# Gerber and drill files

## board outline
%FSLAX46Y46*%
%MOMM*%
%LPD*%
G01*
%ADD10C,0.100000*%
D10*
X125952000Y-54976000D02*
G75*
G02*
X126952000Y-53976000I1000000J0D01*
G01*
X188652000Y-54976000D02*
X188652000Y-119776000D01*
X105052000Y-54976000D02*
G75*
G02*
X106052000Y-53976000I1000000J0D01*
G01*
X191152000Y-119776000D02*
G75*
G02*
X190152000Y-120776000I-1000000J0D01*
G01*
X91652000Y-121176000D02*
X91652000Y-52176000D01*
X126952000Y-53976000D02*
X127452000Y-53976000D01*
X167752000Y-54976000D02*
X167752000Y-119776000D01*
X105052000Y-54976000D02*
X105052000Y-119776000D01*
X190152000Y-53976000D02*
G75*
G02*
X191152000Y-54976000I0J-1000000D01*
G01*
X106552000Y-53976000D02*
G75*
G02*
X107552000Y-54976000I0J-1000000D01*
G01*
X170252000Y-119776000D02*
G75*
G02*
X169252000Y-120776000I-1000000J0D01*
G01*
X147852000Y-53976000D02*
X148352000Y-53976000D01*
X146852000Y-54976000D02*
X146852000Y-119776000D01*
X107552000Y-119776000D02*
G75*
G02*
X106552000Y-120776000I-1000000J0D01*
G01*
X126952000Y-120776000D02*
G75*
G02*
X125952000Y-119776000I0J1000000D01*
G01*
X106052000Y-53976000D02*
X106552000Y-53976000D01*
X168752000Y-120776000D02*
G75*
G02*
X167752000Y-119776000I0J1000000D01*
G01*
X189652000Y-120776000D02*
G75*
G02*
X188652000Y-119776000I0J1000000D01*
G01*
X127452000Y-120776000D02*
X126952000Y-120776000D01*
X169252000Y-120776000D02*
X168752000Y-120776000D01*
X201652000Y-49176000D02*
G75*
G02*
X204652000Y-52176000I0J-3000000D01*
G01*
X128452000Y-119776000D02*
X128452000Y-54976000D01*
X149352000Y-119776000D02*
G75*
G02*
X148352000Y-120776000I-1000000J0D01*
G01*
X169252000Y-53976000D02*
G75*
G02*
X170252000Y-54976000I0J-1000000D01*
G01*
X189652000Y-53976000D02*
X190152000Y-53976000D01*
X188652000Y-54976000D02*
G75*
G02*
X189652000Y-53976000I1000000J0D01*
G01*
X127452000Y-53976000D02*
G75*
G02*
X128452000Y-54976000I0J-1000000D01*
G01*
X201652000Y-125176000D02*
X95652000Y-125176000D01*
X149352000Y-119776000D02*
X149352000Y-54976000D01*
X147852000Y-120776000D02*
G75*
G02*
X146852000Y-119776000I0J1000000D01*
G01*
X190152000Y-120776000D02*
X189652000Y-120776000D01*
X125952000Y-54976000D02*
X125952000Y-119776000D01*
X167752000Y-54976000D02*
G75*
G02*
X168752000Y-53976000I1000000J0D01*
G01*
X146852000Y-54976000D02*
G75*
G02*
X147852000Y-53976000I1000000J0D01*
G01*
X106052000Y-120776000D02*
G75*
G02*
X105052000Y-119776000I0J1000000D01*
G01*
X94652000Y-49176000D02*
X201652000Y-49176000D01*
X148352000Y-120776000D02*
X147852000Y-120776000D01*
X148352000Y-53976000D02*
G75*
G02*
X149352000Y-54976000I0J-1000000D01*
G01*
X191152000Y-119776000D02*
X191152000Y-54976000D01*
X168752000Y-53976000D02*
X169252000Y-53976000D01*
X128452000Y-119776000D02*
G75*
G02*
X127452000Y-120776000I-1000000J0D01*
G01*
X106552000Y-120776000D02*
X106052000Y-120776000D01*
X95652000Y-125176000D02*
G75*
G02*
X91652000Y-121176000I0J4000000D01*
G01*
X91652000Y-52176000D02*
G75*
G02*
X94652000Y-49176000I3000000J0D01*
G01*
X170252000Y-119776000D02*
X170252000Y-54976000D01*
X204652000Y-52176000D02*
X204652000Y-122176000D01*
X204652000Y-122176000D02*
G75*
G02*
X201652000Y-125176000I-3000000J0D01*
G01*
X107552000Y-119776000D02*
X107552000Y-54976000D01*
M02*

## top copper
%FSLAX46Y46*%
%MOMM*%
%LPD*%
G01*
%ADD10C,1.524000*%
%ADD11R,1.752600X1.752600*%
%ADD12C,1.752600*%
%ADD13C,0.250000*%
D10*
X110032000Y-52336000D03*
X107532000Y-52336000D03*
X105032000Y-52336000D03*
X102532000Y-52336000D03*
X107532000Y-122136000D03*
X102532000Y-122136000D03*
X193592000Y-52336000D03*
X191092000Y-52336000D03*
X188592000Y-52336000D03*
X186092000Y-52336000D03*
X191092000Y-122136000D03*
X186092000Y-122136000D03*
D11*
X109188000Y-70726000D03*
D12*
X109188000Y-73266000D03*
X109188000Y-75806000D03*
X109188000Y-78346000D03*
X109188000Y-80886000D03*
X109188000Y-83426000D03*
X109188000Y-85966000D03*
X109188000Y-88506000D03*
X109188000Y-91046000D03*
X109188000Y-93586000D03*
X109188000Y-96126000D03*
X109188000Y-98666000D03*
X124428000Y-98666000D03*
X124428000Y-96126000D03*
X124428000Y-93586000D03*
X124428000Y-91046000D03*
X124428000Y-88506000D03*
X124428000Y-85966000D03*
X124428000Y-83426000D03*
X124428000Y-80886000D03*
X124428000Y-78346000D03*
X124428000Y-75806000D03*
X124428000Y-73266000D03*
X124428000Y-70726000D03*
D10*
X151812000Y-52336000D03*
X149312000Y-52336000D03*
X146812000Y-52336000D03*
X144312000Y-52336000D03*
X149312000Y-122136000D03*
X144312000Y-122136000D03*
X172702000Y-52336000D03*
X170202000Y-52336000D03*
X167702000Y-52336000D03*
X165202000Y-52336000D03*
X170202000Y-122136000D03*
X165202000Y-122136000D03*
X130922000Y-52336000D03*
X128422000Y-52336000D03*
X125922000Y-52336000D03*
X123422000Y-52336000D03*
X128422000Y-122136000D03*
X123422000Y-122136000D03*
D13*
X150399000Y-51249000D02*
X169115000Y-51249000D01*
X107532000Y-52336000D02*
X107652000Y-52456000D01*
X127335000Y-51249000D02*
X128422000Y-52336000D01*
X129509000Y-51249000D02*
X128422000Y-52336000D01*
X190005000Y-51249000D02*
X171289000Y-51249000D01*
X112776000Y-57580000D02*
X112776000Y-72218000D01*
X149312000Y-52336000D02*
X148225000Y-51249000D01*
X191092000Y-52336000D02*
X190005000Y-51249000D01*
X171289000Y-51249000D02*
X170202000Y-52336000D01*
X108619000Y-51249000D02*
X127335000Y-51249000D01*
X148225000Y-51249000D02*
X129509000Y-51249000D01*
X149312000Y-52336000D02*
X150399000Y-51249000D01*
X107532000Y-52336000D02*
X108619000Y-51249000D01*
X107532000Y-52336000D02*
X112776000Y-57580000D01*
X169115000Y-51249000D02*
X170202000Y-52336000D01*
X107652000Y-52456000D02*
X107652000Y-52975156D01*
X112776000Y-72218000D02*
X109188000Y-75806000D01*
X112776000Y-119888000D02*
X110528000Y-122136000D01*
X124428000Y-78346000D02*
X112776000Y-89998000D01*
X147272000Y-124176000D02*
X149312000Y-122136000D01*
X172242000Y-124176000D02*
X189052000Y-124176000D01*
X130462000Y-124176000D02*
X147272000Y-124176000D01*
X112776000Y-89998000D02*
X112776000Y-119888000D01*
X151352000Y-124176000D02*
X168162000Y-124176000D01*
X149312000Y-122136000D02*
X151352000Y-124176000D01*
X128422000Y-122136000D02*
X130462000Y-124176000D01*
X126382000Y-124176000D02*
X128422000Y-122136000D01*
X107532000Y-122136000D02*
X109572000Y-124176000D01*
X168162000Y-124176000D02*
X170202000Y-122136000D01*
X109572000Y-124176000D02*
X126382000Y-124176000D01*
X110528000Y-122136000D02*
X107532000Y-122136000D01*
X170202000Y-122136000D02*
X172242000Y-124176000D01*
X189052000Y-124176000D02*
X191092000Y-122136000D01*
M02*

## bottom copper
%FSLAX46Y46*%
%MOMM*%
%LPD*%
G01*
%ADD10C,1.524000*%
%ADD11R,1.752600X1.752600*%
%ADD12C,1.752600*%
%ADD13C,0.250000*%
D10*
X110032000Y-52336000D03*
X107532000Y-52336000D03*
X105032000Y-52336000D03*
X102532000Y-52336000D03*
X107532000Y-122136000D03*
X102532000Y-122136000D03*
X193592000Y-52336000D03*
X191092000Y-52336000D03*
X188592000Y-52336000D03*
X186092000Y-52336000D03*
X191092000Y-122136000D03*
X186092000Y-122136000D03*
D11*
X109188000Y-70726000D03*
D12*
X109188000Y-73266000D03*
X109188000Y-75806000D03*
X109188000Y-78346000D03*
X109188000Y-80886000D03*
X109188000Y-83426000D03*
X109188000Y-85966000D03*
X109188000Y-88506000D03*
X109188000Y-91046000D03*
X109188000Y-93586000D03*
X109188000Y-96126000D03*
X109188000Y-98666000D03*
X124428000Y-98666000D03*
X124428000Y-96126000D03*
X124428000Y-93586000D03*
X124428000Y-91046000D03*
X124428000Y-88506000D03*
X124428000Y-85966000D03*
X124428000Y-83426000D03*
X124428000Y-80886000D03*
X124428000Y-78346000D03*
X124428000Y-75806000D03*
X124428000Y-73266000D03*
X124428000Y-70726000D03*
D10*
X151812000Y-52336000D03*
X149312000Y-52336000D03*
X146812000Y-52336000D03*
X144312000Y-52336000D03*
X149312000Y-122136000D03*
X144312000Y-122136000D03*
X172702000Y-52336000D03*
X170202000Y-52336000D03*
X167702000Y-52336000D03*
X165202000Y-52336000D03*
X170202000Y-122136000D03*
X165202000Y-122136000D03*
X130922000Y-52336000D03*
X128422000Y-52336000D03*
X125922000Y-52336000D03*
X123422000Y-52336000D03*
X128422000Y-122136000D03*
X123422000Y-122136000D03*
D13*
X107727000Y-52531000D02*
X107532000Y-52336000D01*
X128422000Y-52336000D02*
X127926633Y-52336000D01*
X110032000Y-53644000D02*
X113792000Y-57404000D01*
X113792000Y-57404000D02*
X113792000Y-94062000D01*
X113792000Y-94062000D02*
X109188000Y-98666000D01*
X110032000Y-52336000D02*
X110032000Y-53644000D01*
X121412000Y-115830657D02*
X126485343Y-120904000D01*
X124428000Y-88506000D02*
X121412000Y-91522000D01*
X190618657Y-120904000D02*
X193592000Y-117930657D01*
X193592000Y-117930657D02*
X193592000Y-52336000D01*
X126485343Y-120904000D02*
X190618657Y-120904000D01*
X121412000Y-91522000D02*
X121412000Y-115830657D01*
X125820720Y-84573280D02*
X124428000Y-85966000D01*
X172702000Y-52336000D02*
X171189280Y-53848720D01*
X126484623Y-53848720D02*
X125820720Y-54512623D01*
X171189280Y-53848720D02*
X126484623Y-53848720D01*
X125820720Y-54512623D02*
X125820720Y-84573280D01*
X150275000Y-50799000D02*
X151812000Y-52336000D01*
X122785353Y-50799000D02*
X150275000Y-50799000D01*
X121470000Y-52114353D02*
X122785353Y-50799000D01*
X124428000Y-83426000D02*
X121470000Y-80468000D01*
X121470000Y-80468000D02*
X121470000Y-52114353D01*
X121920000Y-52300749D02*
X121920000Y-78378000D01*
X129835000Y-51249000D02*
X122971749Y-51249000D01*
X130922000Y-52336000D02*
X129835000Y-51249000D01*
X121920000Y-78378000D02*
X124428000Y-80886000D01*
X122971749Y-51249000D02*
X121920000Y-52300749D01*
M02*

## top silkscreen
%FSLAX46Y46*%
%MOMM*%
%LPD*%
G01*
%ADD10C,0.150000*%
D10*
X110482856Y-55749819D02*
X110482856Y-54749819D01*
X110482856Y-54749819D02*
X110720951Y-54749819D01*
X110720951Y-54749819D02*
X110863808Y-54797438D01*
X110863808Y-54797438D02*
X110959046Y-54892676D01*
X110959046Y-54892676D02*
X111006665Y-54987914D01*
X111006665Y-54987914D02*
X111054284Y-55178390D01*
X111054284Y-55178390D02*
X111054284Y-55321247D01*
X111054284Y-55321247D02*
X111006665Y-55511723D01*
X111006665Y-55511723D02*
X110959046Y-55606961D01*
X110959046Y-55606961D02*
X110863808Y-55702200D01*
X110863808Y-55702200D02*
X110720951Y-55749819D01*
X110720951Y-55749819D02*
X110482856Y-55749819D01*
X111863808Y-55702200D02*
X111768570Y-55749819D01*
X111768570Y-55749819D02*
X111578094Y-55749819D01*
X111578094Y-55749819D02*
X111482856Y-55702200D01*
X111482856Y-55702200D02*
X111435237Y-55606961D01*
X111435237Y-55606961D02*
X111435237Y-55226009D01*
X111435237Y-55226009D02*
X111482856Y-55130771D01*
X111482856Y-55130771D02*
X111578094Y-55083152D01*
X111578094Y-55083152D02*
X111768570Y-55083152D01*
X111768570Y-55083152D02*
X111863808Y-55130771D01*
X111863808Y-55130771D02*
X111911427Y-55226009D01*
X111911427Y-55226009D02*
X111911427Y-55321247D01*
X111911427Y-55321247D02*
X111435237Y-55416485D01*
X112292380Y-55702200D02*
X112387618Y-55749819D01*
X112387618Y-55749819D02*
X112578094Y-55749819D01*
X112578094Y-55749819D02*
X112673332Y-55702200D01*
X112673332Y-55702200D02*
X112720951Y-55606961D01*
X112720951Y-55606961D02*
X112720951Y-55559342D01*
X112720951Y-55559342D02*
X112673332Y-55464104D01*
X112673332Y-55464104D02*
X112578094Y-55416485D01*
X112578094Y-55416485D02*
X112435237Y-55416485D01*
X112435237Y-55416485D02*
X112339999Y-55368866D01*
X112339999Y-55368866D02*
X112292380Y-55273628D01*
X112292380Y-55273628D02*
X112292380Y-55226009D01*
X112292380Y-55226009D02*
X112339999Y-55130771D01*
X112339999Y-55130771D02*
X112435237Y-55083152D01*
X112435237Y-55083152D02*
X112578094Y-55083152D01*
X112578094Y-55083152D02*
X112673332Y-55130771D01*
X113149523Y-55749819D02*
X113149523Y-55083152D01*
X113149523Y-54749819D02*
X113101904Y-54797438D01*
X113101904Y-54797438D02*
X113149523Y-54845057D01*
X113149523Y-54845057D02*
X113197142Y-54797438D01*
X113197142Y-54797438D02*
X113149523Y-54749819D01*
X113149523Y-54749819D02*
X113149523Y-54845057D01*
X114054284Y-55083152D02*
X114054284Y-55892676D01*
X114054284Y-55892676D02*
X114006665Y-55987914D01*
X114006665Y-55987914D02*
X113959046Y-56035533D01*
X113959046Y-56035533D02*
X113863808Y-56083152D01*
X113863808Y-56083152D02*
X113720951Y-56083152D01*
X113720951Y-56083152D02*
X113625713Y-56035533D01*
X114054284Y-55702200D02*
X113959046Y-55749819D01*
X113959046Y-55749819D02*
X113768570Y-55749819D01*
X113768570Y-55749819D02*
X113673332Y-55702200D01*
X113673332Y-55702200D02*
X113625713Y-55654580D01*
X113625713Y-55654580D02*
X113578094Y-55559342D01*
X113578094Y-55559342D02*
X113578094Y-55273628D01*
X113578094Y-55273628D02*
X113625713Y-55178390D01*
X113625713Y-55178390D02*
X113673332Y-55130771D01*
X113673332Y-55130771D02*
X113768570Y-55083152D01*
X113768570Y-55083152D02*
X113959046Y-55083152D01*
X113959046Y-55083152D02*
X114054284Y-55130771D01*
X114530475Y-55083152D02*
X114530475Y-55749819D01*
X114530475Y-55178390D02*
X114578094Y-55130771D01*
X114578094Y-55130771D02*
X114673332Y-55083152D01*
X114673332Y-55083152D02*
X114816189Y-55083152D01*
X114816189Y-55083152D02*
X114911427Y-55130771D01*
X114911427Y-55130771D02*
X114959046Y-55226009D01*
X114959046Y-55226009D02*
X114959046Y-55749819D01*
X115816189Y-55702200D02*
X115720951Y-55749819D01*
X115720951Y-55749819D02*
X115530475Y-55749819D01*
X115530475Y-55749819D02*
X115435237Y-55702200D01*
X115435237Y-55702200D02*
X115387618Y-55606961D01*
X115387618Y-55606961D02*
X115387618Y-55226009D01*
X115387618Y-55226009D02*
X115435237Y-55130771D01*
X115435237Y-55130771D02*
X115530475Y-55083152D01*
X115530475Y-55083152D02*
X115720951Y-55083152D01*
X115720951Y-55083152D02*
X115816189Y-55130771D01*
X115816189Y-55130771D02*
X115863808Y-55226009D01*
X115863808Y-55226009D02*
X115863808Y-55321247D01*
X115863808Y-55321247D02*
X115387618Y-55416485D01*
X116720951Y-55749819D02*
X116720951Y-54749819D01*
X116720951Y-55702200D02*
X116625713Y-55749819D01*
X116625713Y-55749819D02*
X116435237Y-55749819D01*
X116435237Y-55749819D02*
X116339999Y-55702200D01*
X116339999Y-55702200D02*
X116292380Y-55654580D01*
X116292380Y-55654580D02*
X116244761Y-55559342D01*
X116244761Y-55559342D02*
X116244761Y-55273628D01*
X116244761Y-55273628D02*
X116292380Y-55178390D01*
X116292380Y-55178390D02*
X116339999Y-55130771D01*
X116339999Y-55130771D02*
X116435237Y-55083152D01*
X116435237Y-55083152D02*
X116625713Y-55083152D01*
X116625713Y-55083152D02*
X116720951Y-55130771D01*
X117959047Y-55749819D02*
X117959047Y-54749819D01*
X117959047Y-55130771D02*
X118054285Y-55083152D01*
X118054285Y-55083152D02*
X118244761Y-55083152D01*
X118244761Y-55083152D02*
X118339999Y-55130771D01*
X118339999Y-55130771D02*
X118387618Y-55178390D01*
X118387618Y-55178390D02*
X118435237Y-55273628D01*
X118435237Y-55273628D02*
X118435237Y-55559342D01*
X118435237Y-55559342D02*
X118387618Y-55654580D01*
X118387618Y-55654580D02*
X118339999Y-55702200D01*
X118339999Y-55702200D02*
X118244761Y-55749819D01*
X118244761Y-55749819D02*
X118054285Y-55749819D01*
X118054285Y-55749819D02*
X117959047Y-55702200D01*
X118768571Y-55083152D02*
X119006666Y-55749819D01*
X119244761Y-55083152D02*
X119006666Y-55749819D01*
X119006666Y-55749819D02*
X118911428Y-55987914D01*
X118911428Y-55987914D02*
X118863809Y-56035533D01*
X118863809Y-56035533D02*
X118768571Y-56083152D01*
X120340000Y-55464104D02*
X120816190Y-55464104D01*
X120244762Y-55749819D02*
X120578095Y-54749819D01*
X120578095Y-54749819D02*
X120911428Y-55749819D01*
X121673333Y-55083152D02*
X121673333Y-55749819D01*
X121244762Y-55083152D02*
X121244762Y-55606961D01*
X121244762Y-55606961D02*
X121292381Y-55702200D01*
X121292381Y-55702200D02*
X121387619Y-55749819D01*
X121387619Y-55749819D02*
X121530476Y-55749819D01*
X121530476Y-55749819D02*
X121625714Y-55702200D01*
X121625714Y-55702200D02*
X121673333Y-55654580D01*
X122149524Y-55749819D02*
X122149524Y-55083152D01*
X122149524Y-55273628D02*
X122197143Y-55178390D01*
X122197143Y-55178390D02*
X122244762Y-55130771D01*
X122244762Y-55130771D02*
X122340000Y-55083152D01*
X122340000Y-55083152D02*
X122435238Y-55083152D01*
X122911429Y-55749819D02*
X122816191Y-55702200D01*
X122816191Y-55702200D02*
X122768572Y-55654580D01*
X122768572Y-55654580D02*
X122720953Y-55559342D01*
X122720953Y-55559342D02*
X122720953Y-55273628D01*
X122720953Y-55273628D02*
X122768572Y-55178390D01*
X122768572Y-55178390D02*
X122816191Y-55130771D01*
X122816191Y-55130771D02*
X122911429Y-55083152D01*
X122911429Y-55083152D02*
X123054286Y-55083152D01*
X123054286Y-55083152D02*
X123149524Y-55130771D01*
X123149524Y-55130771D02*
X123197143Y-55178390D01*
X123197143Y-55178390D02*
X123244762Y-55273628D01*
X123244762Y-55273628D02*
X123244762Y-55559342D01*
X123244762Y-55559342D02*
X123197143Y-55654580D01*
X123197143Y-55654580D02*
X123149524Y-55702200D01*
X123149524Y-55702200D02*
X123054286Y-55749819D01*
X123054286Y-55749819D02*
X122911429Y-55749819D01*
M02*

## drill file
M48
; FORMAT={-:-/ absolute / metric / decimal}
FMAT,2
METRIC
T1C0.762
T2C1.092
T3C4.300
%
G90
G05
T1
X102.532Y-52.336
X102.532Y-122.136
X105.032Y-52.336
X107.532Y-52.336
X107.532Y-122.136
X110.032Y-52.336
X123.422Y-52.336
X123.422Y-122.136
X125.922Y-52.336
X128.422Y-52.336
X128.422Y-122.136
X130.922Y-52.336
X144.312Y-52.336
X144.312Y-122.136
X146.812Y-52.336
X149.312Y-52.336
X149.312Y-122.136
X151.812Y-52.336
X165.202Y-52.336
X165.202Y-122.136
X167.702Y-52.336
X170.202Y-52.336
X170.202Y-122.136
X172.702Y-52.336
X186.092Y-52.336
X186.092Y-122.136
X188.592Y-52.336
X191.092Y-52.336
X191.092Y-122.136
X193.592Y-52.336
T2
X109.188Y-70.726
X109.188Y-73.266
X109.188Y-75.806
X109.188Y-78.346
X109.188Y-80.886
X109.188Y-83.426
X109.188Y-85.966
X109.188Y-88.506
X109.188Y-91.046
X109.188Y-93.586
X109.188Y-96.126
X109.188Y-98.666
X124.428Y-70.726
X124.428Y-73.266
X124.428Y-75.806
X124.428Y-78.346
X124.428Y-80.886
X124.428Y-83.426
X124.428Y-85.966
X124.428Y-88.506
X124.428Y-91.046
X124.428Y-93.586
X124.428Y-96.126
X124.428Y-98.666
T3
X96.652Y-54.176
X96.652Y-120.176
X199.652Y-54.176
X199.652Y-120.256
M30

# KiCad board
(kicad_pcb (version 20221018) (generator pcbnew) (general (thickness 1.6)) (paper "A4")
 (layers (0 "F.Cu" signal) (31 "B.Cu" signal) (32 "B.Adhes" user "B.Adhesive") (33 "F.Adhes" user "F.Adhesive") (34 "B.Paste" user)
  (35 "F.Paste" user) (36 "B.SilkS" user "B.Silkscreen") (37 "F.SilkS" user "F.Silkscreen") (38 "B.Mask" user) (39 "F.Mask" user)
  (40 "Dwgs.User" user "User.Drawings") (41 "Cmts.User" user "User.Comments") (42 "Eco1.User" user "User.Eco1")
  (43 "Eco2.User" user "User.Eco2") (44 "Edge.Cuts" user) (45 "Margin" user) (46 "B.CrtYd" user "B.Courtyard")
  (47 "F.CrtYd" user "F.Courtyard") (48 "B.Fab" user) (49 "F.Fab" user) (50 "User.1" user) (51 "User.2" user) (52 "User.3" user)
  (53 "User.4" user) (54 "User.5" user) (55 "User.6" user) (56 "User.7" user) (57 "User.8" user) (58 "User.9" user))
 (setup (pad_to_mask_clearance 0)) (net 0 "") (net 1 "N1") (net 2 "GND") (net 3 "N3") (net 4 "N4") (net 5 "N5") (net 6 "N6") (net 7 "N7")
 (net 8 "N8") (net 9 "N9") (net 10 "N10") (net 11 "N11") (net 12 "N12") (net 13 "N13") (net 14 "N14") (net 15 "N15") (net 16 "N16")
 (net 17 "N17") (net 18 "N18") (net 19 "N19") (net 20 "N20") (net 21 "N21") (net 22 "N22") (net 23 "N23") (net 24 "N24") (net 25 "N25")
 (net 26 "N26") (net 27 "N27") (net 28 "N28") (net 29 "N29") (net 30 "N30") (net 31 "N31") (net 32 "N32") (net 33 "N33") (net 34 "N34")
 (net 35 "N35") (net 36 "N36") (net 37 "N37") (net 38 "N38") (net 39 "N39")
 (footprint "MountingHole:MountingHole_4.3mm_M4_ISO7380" (layer "F.Cu") (at 199.652 120.256)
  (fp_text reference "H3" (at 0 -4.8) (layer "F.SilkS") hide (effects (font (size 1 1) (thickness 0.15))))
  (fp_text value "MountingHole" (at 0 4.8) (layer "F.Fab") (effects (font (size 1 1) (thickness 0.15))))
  (pad "" np_thru_hole circle (at 0 0) (size 4.3 4.3) (drill 4.3) (layers "*.Cu" "*.Mask")))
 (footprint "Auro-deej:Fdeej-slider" (layer "F.Cu") (at 105.632 87.236 -90)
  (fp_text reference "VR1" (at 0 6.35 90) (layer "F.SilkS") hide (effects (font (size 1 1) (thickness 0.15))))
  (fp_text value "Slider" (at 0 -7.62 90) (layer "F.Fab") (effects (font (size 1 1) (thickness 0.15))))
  (pad "1" thru_hole circle (at -34.9 -4.4 270) (size 1.524 1.524) (drill 0.762) (layers "*.Cu" "*.Mask") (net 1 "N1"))
  (pad "2" thru_hole circle (at -34.9 -1.9 270) (size 1.524 1.524) (drill 0.762) (layers "*.Cu" "*.Mask") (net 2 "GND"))
  (pad "3" thru_hole circle (at -34.9 0.6 270) (size 1.524 1.524) (drill 0.762) (layers "*.Cu" "*.Mask") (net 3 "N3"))
  (pad "4" thru_hole circle (at -34.9 3.1 270) (size 1.524 1.524) (drill 0.762) (layers "*.Cu" "*.Mask") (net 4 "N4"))
  (pad "5" thru_hole circle (at 34.9 -1.9 270) (size 1.524 1.524) (drill 0.762) (layers "*.Cu" "*.Mask") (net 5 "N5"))
  (pad "6" thru_hole circle (at 34.9 3.1 270) (size 1.524 1.524) (drill 0.762) (layers "*.Cu" "*.Mask") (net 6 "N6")))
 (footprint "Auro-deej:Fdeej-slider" (layer "F.Cu") (at 189.192 87.236 -90)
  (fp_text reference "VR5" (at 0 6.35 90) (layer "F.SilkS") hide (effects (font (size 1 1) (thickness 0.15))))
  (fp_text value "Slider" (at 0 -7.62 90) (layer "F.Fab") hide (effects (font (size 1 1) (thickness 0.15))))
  (pad "1" thru_hole circle (at -34.9 -4.4 270) (size 1.524 1.524) (drill 0.762) (layers "*.Cu" "*.Mask") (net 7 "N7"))
  (pad "2" thru_hole circle (at -34.9 -1.9 270) (size 1.524 1.524) (drill 0.762) (layers "*.Cu" "*.Mask") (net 2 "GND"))
  (pad "3" thru_hole circle (at -34.9 0.6 270) (size 1.524 1.524) (drill 0.762) (layers "*.Cu" "*.Mask") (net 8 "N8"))
  (pad "4" thru_hole circle (at -34.9 3.1 270) (size 1.524 1.524) (drill 0.762) (layers "*.Cu" "*.Mask") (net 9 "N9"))
  (pad "5" thru_hole circle (at 34.9 -1.9 270) (size 1.524 1.524) (drill 0.762) (layers "*.Cu" "*.Mask") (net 5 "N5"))
  (pad "6" thru_hole circle (at 34.9 3.1 270) (size 1.524 1.524) (drill 0.762) (layers "*.Cu" "*.Mask") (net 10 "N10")))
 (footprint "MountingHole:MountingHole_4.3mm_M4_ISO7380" (layer "F.Cu") (at 199.652 54.176)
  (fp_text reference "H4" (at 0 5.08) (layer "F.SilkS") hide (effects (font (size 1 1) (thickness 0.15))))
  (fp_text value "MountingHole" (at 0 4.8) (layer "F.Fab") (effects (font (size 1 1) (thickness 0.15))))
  (pad "" np_thru_hole circle (at 0 0) (size 4.3 4.3) (drill 4.3) (layers "*.Cu" "*.Mask")))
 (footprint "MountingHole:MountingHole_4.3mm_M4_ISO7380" (layer "F.Cu") (at 96.652 120.176)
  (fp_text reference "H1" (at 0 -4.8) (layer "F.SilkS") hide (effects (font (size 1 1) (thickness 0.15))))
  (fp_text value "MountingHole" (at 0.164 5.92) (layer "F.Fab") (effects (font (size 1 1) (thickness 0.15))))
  (pad "" np_thru_hole circle (at 0 0) (size 4.3 4.3) (drill 4.3) (layers "*.Cu" "*.Mask")))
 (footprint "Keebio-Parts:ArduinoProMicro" (layer "F.Cu") (at 116.808 84.696 -90)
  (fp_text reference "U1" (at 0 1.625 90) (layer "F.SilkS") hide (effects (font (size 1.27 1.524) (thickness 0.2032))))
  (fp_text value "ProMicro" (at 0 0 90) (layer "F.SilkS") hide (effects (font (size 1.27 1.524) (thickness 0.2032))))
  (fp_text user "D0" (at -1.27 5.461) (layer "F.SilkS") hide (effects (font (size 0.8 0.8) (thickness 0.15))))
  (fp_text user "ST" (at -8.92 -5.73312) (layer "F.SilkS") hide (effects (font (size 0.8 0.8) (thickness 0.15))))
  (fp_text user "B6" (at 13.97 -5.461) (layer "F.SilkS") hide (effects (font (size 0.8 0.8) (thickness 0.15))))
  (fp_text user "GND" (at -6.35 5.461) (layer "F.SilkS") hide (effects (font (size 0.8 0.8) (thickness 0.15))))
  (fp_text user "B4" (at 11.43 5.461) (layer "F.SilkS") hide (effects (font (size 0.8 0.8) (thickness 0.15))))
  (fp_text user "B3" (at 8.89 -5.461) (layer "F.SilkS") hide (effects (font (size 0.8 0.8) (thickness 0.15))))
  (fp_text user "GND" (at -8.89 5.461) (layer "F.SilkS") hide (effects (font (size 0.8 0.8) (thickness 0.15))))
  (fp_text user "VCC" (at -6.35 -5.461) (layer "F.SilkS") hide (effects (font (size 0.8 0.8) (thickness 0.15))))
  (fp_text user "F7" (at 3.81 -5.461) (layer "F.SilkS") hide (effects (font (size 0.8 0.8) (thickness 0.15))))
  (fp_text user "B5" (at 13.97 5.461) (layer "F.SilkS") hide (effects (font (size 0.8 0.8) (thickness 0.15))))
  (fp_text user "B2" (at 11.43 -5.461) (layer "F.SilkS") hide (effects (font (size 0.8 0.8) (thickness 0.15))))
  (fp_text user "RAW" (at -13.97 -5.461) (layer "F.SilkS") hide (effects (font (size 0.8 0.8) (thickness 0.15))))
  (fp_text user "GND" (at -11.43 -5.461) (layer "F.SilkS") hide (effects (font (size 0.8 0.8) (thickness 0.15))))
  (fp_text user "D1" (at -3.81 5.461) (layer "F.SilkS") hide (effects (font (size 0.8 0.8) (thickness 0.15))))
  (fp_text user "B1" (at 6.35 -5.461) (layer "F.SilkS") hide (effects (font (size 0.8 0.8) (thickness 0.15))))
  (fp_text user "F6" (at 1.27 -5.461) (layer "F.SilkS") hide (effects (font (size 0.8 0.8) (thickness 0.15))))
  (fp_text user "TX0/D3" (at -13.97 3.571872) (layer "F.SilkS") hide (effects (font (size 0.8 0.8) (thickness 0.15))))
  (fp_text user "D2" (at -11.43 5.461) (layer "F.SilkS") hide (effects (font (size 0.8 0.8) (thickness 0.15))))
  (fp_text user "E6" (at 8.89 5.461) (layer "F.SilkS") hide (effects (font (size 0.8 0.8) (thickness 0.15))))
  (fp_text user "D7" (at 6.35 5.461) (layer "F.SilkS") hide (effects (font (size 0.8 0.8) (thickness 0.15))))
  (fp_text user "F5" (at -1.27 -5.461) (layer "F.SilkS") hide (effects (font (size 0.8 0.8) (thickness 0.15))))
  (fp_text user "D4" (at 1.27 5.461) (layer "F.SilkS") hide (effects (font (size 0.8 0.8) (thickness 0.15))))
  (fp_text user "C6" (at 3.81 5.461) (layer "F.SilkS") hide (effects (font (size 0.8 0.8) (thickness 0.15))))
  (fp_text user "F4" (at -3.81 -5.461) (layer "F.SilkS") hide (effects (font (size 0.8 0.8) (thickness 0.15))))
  (pad "1" thru_hole rect (at -13.97 7.62 270) (size 1.7526 1.7526) (drill 1.0922) (layers "*.Cu" "*.Mask") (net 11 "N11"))
  (pad "2" thru_hole circle (at -11.43 7.62 270) (size 1.7526 1.7526) (drill 1.0922) (layers "*.Cu" "*.Mask") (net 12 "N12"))
  (pad "3" thru_hole circle (at -8.89 7.62 270) (size 1.7526 1.7526) (drill 1.0922) (layers "*.Cu" "*.Mask") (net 2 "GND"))
  (pad "4" thru_hole circle (at -6.35 7.62 270) (size 1.7526 1.7526) (drill 1.0922) (layers "*.Cu" "*.Mask") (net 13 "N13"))
  (pad "5" thru_hole circle (at -3.81 7.62 270) (size 1.7526 1.7526) (drill 1.0922) (layers "*.Cu" "*.Mask") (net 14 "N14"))
  (pad "6" thru_hole circle (at -1.27 7.62 270) (size 1.7526 1.7526) (drill 1.0922) (layers "*.Cu" "*.Mask") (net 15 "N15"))
  (pad "7" thru_hole circle (at 1.27 7.62 270) (size 1.7526 1.7526) (drill 1.0922) (layers "*.Cu" "*.Mask") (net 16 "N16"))
  (pad "8" thru_hole circle (at 3.81 7.62 270) (size 1.7526 1.7526) (drill 1.0922) (layers "*.Cu" "*.Mask") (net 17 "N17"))
  (pad "9" thru_hole circle (at 6.35 7.62 270) (size 1.7526 1.7526) (drill 1.0922) (layers "*.Cu" "*.Mask") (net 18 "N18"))
  (pad "10" thru_hole circle (at 8.89 7.62 270) (size 1.7526 1.7526) (drill 1.0922) (layers "*.Cu" "*.Mask") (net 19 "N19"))
  (pad "11" thru_hole circle (at 11.43 7.62 270) (size 1.7526 1.7526) (drill 1.0922) (layers "*.Cu" "*.Mask") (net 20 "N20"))
  (pad "12" thru_hole circle (at 13.97 7.62 270) (size 1.7526 1.7526) (drill 1.0922) (layers "*.Cu" "*.Mask") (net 1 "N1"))
  (pad "13" thru_hole circle (at 13.97 -7.62 270) (size 1.7526 1.7526) (drill 1.0922) (layers "*.Cu" "*.Mask") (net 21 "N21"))
  (pad "14" thru_hole circle (at 11.43 -7.62 270) (size 1.7526 1.7526) (drill 1.0922) (layers "*.Cu" "*.Mask") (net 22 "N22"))
  (pad "15" thru_hole circle (at 8.89 -7.62 270) (size 1.7526 1.7526) (drill 1.0922) (layers "*.Cu" "*.Mask") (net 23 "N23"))
  (pad "16" thru_hole circle (at 6.35 -7.62 270) (size 1.7526 1.7526) (drill 1.0922) (layers "*.Cu" "*.Mask") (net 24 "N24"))
  (pad "17" thru_hole circle (at 3.81 -7.62 270) (size 1.7526 1.7526) (drill 1.0922) (layers "*.Cu" "*.Mask") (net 7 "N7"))
  (pad "18" thru_hole circle (at 1.27 -7.62 270) (size 1.7526 1.7526) (drill 1.0922) (layers "*.Cu" "*.Mask") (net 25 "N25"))
  (pad "19" thru_hole circle (at -1.27 -7.62 270) (size 1.7526 1.7526) (drill 1.0922) (layers "*.Cu" "*.Mask") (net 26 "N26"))
  (pad "20" thru_hole circle (at -3.81 -7.62 270) (size 1.7526 1.7526) (drill 1.0922) (layers "*.Cu" "*.Mask") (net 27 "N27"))
  (pad "21" thru_hole circle (at -6.35 -7.62 270) (size 1.7526 1.7526) (drill 1.0922) (layers "*.Cu" "*.Mask") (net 5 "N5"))
  (pad "22" thru_hole circle (at -8.89 -7.62 270) (size 1.7526 1.7526) (drill 1.0922) (layers "*.Cu" "*.Mask") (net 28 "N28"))
  (pad "23" thru_hole circle (at -11.43 -7.62 270) (size 1.7526 1.7526) (drill 1.0922) (layers "*.Cu" "*.Mask") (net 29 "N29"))
  (pad "24" thru_hole circle (at -13.97 -7.62 270) (size 1.7526 1.7526) (drill 1.0922) (layers "*.Cu" "*.Mask") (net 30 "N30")))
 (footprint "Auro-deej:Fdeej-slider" (layer "F.Cu") (at 147.412 87.236 -90)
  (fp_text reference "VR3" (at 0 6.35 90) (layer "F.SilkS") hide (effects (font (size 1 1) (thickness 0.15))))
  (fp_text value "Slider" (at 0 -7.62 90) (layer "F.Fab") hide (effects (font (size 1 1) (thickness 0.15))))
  (pad "1" thru_hole circle (at -34.9 -4.4 270) (size 1.524 1.524) (drill 0.762) (layers "*.Cu" "*.Mask") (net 26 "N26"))
  (pad "2" thru_hole circle (at -34.9 -1.9 270) (size 1.524 1.524) (drill 0.762) (layers "*.Cu" "*.Mask") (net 2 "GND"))
  (pad "3" thru_hole circle (at -34.9 0.6 270) (size 1.524 1.524) (drill 0.762) (layers "*.Cu" "*.Mask") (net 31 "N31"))
  (pad "4" thru_hole circle (at -34.9 3.1 270) (size 1.524 1.524) (drill 0.762) (layers "*.Cu" "*.Mask") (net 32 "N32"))
  (pad "5" thru_hole circle (at 34.9 -1.9 270) (size 1.524 1.524) (drill 0.762) (layers "*.Cu" "*.Mask") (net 5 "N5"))
  (pad "6" thru_hole circle (at 34.9 3.1 270) (size 1.524 1.524) (drill 0.762) (layers "*.Cu" "*.Mask") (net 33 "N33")))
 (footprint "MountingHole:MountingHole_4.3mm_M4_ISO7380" (layer "F.Cu") (at 96.652 54.176)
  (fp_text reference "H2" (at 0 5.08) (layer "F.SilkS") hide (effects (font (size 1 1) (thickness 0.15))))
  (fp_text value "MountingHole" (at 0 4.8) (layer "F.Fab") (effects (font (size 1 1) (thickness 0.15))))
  (pad "" np_thru_hole circle (at 0 0) (size 4.3 4.3) (drill 4.3) (layers "*.Cu" "*.Mask")))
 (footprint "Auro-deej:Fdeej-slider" (layer "F.Cu") (at 168.302 87.236 -90)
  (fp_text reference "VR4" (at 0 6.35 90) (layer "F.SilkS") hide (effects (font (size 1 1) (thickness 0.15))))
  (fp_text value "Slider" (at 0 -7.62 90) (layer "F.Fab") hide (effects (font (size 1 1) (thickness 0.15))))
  (pad "1" thru_hole circle (at -34.9 -4.4 270) (size 1.524 1.524) (drill 0.762) (layers "*.Cu" "*.Mask") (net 25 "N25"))
  (pad "2" thru_hole circle (at -34.9 -1.9 270) (size 1.524 1.524) (drill 0.762) (layers "*.Cu" "*.Mask") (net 2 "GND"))
  (pad "3" thru_hole circle (at -34.9 0.6 270) (size 1.524 1.524) (drill 0.762) (layers "*.Cu" "*.Mask") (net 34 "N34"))
  (pad "4" thru_hole circle (at -34.9 3.1 270) (size 1.524 1.524) (drill 0.762) (layers "*.Cu" "*.Mask") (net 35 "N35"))
  (pad "5" thru_hole circle (at 34.9 -1.9 270) (size 1.524 1.524) (drill 0.762) (layers "*.Cu" "*.Mask") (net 5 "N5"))
  (pad "6" thru_hole circle (at 34.9 3.1 270) (size 1.524 1.524) (drill 0.762) (layers "*.Cu" "*.Mask") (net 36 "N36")))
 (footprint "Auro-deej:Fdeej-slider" (layer "F.Cu") (at 126.522 87.236 -90)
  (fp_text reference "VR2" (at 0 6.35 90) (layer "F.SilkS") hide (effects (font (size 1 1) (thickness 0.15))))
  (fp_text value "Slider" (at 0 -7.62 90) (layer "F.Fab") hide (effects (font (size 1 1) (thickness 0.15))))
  (pad "1" thru_hole circle (at -34.9 -4.4 270) (size 1.524 1.524) (drill 0.762) (layers "*.Cu" "*.Mask") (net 27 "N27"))
  (pad "2" thru_hole circle (at -34.9 -1.9 270) (size 1.524 1.524) (drill 0.762) (layers "*.Cu" "*.Mask") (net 2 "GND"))
  (pad "3" thru_hole circle (at -34.9 0.6 270) (size 1.524 1.524) (drill 0.762) (layers "*.Cu" "*.Mask") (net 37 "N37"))
  (pad "4" thru_hole circle (at -34.9 3.1 270) (size 1.524 1.524) (drill 0.762) (layers "*.Cu" "*.Mask") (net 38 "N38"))
  (pad "5" thru_hole circle (at 34.9 -1.9 270) (size 1.524 1.524) (drill 0.762) (layers "*.Cu" "*.Mask") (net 5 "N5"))
  (pad "6" thru_hole circle (at 34.9 3.1 270) (size 1.524 1.524) (drill 0.762) (layers "*.Cu" "*.Mask") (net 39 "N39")))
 (gr_arc (start 125.952 54.976) (mid 126.244893 54.268893) (end 126.952 53.976) (stroke (width 0.1) (type solid)) (layer "Edge.Cuts"))
 (gr_line (start 188.652 54.976) (end 188.652 119.776) (stroke (width 0.1) (type solid)) (layer "Edge.Cuts"))
 (gr_arc (start 105.052 54.976) (mid 105.344893 54.268893) (end 106.052 53.976) (stroke (width 0.1) (type solid)) (layer "Edge.Cuts"))
 (gr_arc (start 191.152 119.776) (mid 190.859107 120.483107) (end 190.152 120.776) (stroke (width 0.1) (type solid)) (layer "Edge.Cuts"))
 (gr_line (start 91.652 121.176) (end 91.652 52.176) (stroke (width 0.1) (type solid)) (layer "Edge.Cuts"))
 (gr_line (start 126.952 53.976) (end 127.452 53.976) (stroke (width 0.1) (type solid)) (layer "Edge.Cuts"))
 (gr_line (start 167.752 54.976) (end 167.752 119.776) (stroke (width 0.1) (type solid)) (layer "Edge.Cuts"))
 (gr_line (start 105.052 54.976) (end 105.052 119.776) (stroke (width 0.1) (type solid)) (layer "Edge.Cuts"))
 (gr_arc (start 190.152 53.976) (mid 190.859107 54.268893) (end 191.152 54.976) (stroke (width 0.1) (type solid)) (layer "Edge.Cuts"))
 (gr_arc (start 106.552 53.976) (mid 107.259107 54.268893) (end 107.552 54.976) (stroke (width 0.1) (type solid)) (layer "Edge.Cuts"))
 (gr_arc (start 170.252 119.776) (mid 169.959107 120.483107) (end 169.252 120.776) (stroke (width 0.1) (type solid)) (layer "Edge.Cuts"))
 (gr_line (start 147.852 53.976) (end 148.352 53.976) (stroke (width 0.1) (type solid)) (layer "Edge.Cuts"))
 (gr_line (start 146.852 54.976) (end 146.852 119.776) (stroke (width 0.1) (type solid)) (layer "Edge.Cuts"))
 (gr_arc (start 107.552 119.776) (mid 107.259107 120.483107) (end 106.552 120.776) (stroke (width 0.1) (type solid)) (layer "Edge.Cuts"))
 (gr_arc (start 126.952 120.776) (mid 126.244893 120.483107) (end 125.952 119.776) (stroke (width 0.1) (type solid)) (layer "Edge.Cuts"))
 (gr_line (start 106.052 53.976) (end 106.552 53.976) (stroke (width 0.1) (type solid)) (layer "Edge.Cuts"))
 (gr_arc (start 168.752 120.776) (mid 168.044893 120.483107) (end 167.752 119.776) (stroke (width 0.1) (type solid)) (layer "Edge.Cuts"))
 (gr_arc (start 189.652 120.776) (mid 188.944893 120.483107) (end 188.652 119.776) (stroke (width 0.1) (type solid)) (layer "Edge.Cuts"))
 (gr_line (start 127.452 120.776) (end 126.952 120.776) (stroke (width 0.1) (type solid)) (layer "Edge.Cuts"))
 (gr_line (start 169.252 120.776) (end 168.752 120.776) (stroke (width 0.1) (type solid)) (layer "Edge.Cuts"))
 (gr_arc (start 201.652 49.176) (mid 203.77332 50.05468) (end 204.652 52.176) (stroke (width 0.1) (type solid)) (layer "Edge.Cuts"))
 (gr_line (start 128.452 119.776) (end 128.452 54.976) (stroke (width 0.1) (type solid)) (layer "Edge.Cuts"))
 (gr_arc (start 149.352 119.776) (mid 149.059107 120.483107) (end 148.352 120.776) (stroke (width 0.1) (type solid)) (layer "Edge.Cuts"))
 (gr_arc (start 169.252 53.976) (mid 169.959107 54.268893) (end 170.252 54.976) (stroke (width 0.1) (type solid)) (layer "Edge.Cuts"))
 (gr_line (start 189.652 53.976) (end 190.152 53.976) (stroke (width 0.1) (type solid)) (layer "Edge.Cuts"))
 (gr_arc (start 188.652 54.976) (mid 188.944893 54.268893) (end 189.652 53.976) (stroke (width 0.1) (type solid)) (layer "Edge.Cuts"))
 (gr_arc (start 127.452 53.976) (mid 128.159107 54.268893) (end 128.452 54.976) (stroke (width 0.1) (type solid)) (layer "Edge.Cuts"))
 (gr_line (start 201.652 125.176) (end 95.652 125.176) (stroke (width 0.1) (type solid)) (layer "Edge.Cuts"))
 (gr_line (start 149.352 119.776) (end 149.352 54.976) (stroke (width 0.1) (type solid)) (layer "Edge.Cuts"))
 (gr_arc (start 147.852 120.776) (mid 147.144893 120.483107) (end 146.852 119.776) (stroke (width 0.1) (type solid)) (layer "Edge.Cuts"))
 (gr_line (start 190.152 120.776) (end 189.652 120.776) (stroke (width 0.1) (type solid)) (layer "Edge.Cuts"))
 (gr_line (start 125.952 54.976) (end 125.952 119.776) (stroke (width 0.1) (type solid)) (layer "Edge.Cuts"))
 (gr_arc (start 167.752 54.976) (mid 168.044893 54.268893) (end 168.752 53.976) (stroke (width 0.1) (type solid)) (layer "Edge.Cuts"))
 (gr_arc (start 146.852 54.976) (mid 147.144893 54.268893) (end 147.852 53.976) (stroke (width 0.1) (type solid)) (layer "Edge.Cuts"))
 (gr_arc (start 106.052 120.776) (mid 105.344893 120.483107) (end 105.052 119.776) (stroke (width 0.1) (type solid)) (layer "Edge.Cuts"))
 (gr_line (start 94.652 49.176) (end 201.652 49.176) (stroke (width 0.1) (type solid)) (layer "Edge.Cuts"))
 (gr_line (start 148.352 120.776) (end 147.852 120.776) (stroke (width 0.1) (type solid)) (layer "Edge.Cuts"))
 (gr_arc (start 148.352 53.976) (mid 149.059107 54.268893) (end 149.352 54.976) (stroke (width 0.1) (type solid)) (layer "Edge.Cuts"))
 (gr_line (start 191.152 119.776) (end 191.152 54.976) (stroke (width 0.1) (type solid)) (layer "Edge.Cuts"))
 (gr_line (start 168.752 53.976) (end 169.252 53.976) (stroke (width 0.1) (type solid)) (layer "Edge.Cuts"))
 (gr_arc (start 128.452 119.776) (mid 128.159107 120.483107) (end 127.452 120.776) (stroke (width 0.1) (type solid)) (layer "Edge.Cuts"))
 (gr_line (start 106.552 120.776) (end 106.052 120.776) (stroke (width 0.1) (type solid)) (layer "Edge.Cuts"))
 (gr_arc (start 95.652 125.176) (mid 92.823573 124.004427) (end 91.652 121.176) (stroke (width 0.1) (type solid)) (layer "Edge.Cuts"))
 (gr_arc (start 91.652 52.176) (mid 92.53068 50.05468) (end 94.652 49.176) (stroke (width 0.1) (type solid)) (layer "Edge.Cuts"))
 (gr_line (start 170.252 119.776) (end 170.252 54.976) (stroke (width 0.1) (type solid)) (layer "Edge.Cuts"))
 (gr_line (start 204.652 52.176) (end 204.652 122.176) (stroke (width 0.1) (type solid)) (layer "Edge.Cuts"))
 (gr_arc (start 204.652 122.176) (mid 203.77332 124.29732) (end 201.652 125.176) (stroke (width 0.1) (type solid)) (layer "Edge.Cuts"))
 (gr_line (start 107.552 119.776) (end 107.552 54.976) (stroke (width 0.1) (type solid)) (layer "Edge.Cuts"))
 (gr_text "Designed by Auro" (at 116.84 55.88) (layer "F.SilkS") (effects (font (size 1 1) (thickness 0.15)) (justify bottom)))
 (segment (start 150.399 51.249) (end 169.115 51.249) (width 0.25) (layer "F.Cu") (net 2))
 (segment (start 107.532 52.336) (end 107.652 52.456) (width 0.25) (layer "F.Cu") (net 2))
 (segment (start 127.335 51.249) (end 128.422 52.336) (width 0.25) (layer "F.Cu") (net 2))
 (segment (start 129.509 51.249) (end 128.422 52.336) (width 0.25) (layer "F.Cu") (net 2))
 (segment (start 190.005 51.249) (end 171.289 51.249) (width 0.25) (layer "F.Cu") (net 2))
 (segment (start 112.776 57.58) (end 112.776 72.218) (width 0.25) (layer "F.Cu") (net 2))
 (segment (start 149.312 52.336) (end 148.225 51.249) (width 0.25) (layer "F.Cu") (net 2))
 (segment (start 191.092 52.336) (end 190.005 51.249) (width 0.25) (layer "F.Cu") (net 2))
 (segment (start 171.289 51.249) (end 170.202 52.336) (width 0.25) (layer "F.Cu") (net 2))
 (segment (start 108.619 51.249) (end 127.335 51.249) (width 0.25) (layer "F.Cu") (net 2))
 (segment (start 148.225 51.249) (end 129.509 51.249) (width 0.25) (layer "F.Cu") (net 2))
 (segment (start 149.312 52.336) (end 150.399 51.249) (width 0.25) (layer "F.Cu") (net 2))
 (segment (start 107.532 52.336) (end 108.619 51.249) (width 0.25) (layer "F.Cu") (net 2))
 (segment (start 107.532 52.336) (end 112.776 57.58) (width 0.25) (layer "F.Cu") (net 2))
 (segment (start 169.115 51.249) (end 170.202 52.336) (width 0.25) (layer "F.Cu") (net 2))
 (segment (start 107.652 52.456) (end 107.652 52.975156) (width 0.25) (layer "F.Cu") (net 2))
 (segment (start 112.776 72.218) (end 109.188 75.806) (width 0.25) (layer "F.Cu") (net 2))
 (segment (start 107.727 52.531) (end 107.532 52.336) (width 0.25) (layer "B.Cu") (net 2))
 (segment (start 128.422 52.336) (end 127.926633 52.336) (width 0.25) (layer "B.Cu") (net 2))
 (segment (start 110.032 53.644) (end 113.792 57.404) (width 0.25) (layer "B.Cu") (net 1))
 (segment (start 113.792 57.404) (end 113.792 94.062) (width 0.25) (layer "B.Cu") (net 1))
 (segment (start 113.792 94.062) (end 109.188 98.666) (width 0.25) (layer "B.Cu") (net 1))
 (segment (start 110.032 52.336) (end 110.032 53.644) (width 0.25) (layer "B.Cu") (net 1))
 (segment (start 121.412 115.830657) (end 126.485343 120.904) (width 0.25) (layer "B.Cu") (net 7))
 (segment (start 124.428 88.506) (end 121.412 91.522) (width 0.25) (layer "B.Cu") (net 7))
 (segment (start 190.618657 120.904) (end 193.592 117.930657) (width 0.25) (layer "B.Cu") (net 7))
 (segment (start 193.592 117.930657) (end 193.592 52.336) (width 0.25) (layer "B.Cu") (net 7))
 (segment (start 126.485343 120.904) (end 190.618657 120.904) (width 0.25) (layer "B.Cu") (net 7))
 (segment (start 121.412 91.522) (end 121.412 115.830657) (width 0.25) (layer "B.Cu") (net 7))
 (segment (start 125.82072 84.57328) (end 124.428 85.966) (width 0.25) (layer "B.Cu") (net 25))
 (segment (start 172.702 52.336) (end 171.18928 53.84872) (width 0.25) (layer "B.Cu") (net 25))
 (segment (start 126.484623 53.84872) (end 125.82072 54.512623) (width 0.25) (layer "B.Cu") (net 25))
 (segment (start 171.18928 53.84872) (end 126.484623 53.84872) (width 0.25) (layer "B.Cu") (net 25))
 (segment (start 125.82072 54.512623) (end 125.82072 84.57328) (width 0.25) (layer "B.Cu") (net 25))
 (segment (start 150.275 50.799) (end 151.812 52.336) (width 0.25) (layer "B.Cu") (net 26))
 (segment (start 122.785353 50.799) (end 150.275 50.799) (width 0.25) (layer "B.Cu") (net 26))
 (segment (start 121.47 52.114353) (end 122.785353 50.799) (width 0.25) (layer "B.Cu") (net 26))
 (segment (start 124.428 83.426) (end 121.47 80.468) (width 0.25) (layer "B.Cu") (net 26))
 (segment (start 121.47 80.468) (end 121.47 52.114353) (width 0.25) (layer "B.Cu") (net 26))
 (segment (start 121.92 52.300749) (end 121.92 78.378) (width 0.25) (layer "B.Cu") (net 27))
 (segment (start 129.835 51.249) (end 122.971749 51.249) (width 0.25) (layer "B.Cu") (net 27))
 (segment (start 130.922 52.336) (end 129.835 51.249) (width 0.25) (layer "B.Cu") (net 27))
 (segment (start 121.92 78.378) (end 124.428 80.886) (width 0.25) (layer "B.Cu") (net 27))
 (segment (start 122.971749 51.249) (end 121.92 52.300749) (width 0.25) (layer "B.Cu") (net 27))
 (segment (start 112.776 119.888) (end 110.528 122.136) (width 0.25) (layer "F.Cu") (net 5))
 (segment (start 124.428 78.346) (end 112.776 89.998) (width 0.25) (layer "F.Cu") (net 5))
 (segment (start 147.272 124.176) (end 149.312 122.136) (width 0.25) (layer "F.Cu") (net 5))
 (segment (start 172.242 124.176) (end 189.052 124.176) (width 0.25) (layer "F.Cu") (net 5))
 (segment (start 130.462 124.176) (end 147.272 124.176) (width 0.25) (layer "F.Cu") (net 5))
 (segment (start 112.776 89.998) (end 112.776 119.888) (width 0.25) (layer "F.Cu") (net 5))
 (segment (start 151.352 124.176) (end 168.162 124.176) (width 0.25) (layer "F.Cu") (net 5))
 (segment (start 149.312 122.136) (end 151.352 124.176) (width 0.25) (layer "F.Cu") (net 5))
 (segment (start 128.422 122.136) (end 130.462 124.176) (width 0.25) (layer "F.Cu") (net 5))
 (segment (start 126.382 124.176) (end 128.422 122.136) (width 0.25) (layer "F.Cu") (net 5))
 (segment (start 107.532 122.136) (end 109.572 124.176) (width 0.25) (layer "F.Cu") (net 5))
 (segment (start 168.162 124.176) (end 170.202 122.136) (width 0.25) (layer "F.Cu") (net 5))
 (segment (start 109.572 124.176) (end 126.382 124.176) (width 0.25) (layer "F.Cu") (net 5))
 (segment (start 110.528 122.136) (end 107.532 122.136) (width 0.25) (layer "F.Cu") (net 5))
 (segment (start 170.202 122.136) (end 172.242 124.176) (width 0.25) (layer "F.Cu") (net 5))
 (segment (start 189.052 124.176) (end 191.092 122.136) (width 0.25) (layer "F.Cu") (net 5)))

